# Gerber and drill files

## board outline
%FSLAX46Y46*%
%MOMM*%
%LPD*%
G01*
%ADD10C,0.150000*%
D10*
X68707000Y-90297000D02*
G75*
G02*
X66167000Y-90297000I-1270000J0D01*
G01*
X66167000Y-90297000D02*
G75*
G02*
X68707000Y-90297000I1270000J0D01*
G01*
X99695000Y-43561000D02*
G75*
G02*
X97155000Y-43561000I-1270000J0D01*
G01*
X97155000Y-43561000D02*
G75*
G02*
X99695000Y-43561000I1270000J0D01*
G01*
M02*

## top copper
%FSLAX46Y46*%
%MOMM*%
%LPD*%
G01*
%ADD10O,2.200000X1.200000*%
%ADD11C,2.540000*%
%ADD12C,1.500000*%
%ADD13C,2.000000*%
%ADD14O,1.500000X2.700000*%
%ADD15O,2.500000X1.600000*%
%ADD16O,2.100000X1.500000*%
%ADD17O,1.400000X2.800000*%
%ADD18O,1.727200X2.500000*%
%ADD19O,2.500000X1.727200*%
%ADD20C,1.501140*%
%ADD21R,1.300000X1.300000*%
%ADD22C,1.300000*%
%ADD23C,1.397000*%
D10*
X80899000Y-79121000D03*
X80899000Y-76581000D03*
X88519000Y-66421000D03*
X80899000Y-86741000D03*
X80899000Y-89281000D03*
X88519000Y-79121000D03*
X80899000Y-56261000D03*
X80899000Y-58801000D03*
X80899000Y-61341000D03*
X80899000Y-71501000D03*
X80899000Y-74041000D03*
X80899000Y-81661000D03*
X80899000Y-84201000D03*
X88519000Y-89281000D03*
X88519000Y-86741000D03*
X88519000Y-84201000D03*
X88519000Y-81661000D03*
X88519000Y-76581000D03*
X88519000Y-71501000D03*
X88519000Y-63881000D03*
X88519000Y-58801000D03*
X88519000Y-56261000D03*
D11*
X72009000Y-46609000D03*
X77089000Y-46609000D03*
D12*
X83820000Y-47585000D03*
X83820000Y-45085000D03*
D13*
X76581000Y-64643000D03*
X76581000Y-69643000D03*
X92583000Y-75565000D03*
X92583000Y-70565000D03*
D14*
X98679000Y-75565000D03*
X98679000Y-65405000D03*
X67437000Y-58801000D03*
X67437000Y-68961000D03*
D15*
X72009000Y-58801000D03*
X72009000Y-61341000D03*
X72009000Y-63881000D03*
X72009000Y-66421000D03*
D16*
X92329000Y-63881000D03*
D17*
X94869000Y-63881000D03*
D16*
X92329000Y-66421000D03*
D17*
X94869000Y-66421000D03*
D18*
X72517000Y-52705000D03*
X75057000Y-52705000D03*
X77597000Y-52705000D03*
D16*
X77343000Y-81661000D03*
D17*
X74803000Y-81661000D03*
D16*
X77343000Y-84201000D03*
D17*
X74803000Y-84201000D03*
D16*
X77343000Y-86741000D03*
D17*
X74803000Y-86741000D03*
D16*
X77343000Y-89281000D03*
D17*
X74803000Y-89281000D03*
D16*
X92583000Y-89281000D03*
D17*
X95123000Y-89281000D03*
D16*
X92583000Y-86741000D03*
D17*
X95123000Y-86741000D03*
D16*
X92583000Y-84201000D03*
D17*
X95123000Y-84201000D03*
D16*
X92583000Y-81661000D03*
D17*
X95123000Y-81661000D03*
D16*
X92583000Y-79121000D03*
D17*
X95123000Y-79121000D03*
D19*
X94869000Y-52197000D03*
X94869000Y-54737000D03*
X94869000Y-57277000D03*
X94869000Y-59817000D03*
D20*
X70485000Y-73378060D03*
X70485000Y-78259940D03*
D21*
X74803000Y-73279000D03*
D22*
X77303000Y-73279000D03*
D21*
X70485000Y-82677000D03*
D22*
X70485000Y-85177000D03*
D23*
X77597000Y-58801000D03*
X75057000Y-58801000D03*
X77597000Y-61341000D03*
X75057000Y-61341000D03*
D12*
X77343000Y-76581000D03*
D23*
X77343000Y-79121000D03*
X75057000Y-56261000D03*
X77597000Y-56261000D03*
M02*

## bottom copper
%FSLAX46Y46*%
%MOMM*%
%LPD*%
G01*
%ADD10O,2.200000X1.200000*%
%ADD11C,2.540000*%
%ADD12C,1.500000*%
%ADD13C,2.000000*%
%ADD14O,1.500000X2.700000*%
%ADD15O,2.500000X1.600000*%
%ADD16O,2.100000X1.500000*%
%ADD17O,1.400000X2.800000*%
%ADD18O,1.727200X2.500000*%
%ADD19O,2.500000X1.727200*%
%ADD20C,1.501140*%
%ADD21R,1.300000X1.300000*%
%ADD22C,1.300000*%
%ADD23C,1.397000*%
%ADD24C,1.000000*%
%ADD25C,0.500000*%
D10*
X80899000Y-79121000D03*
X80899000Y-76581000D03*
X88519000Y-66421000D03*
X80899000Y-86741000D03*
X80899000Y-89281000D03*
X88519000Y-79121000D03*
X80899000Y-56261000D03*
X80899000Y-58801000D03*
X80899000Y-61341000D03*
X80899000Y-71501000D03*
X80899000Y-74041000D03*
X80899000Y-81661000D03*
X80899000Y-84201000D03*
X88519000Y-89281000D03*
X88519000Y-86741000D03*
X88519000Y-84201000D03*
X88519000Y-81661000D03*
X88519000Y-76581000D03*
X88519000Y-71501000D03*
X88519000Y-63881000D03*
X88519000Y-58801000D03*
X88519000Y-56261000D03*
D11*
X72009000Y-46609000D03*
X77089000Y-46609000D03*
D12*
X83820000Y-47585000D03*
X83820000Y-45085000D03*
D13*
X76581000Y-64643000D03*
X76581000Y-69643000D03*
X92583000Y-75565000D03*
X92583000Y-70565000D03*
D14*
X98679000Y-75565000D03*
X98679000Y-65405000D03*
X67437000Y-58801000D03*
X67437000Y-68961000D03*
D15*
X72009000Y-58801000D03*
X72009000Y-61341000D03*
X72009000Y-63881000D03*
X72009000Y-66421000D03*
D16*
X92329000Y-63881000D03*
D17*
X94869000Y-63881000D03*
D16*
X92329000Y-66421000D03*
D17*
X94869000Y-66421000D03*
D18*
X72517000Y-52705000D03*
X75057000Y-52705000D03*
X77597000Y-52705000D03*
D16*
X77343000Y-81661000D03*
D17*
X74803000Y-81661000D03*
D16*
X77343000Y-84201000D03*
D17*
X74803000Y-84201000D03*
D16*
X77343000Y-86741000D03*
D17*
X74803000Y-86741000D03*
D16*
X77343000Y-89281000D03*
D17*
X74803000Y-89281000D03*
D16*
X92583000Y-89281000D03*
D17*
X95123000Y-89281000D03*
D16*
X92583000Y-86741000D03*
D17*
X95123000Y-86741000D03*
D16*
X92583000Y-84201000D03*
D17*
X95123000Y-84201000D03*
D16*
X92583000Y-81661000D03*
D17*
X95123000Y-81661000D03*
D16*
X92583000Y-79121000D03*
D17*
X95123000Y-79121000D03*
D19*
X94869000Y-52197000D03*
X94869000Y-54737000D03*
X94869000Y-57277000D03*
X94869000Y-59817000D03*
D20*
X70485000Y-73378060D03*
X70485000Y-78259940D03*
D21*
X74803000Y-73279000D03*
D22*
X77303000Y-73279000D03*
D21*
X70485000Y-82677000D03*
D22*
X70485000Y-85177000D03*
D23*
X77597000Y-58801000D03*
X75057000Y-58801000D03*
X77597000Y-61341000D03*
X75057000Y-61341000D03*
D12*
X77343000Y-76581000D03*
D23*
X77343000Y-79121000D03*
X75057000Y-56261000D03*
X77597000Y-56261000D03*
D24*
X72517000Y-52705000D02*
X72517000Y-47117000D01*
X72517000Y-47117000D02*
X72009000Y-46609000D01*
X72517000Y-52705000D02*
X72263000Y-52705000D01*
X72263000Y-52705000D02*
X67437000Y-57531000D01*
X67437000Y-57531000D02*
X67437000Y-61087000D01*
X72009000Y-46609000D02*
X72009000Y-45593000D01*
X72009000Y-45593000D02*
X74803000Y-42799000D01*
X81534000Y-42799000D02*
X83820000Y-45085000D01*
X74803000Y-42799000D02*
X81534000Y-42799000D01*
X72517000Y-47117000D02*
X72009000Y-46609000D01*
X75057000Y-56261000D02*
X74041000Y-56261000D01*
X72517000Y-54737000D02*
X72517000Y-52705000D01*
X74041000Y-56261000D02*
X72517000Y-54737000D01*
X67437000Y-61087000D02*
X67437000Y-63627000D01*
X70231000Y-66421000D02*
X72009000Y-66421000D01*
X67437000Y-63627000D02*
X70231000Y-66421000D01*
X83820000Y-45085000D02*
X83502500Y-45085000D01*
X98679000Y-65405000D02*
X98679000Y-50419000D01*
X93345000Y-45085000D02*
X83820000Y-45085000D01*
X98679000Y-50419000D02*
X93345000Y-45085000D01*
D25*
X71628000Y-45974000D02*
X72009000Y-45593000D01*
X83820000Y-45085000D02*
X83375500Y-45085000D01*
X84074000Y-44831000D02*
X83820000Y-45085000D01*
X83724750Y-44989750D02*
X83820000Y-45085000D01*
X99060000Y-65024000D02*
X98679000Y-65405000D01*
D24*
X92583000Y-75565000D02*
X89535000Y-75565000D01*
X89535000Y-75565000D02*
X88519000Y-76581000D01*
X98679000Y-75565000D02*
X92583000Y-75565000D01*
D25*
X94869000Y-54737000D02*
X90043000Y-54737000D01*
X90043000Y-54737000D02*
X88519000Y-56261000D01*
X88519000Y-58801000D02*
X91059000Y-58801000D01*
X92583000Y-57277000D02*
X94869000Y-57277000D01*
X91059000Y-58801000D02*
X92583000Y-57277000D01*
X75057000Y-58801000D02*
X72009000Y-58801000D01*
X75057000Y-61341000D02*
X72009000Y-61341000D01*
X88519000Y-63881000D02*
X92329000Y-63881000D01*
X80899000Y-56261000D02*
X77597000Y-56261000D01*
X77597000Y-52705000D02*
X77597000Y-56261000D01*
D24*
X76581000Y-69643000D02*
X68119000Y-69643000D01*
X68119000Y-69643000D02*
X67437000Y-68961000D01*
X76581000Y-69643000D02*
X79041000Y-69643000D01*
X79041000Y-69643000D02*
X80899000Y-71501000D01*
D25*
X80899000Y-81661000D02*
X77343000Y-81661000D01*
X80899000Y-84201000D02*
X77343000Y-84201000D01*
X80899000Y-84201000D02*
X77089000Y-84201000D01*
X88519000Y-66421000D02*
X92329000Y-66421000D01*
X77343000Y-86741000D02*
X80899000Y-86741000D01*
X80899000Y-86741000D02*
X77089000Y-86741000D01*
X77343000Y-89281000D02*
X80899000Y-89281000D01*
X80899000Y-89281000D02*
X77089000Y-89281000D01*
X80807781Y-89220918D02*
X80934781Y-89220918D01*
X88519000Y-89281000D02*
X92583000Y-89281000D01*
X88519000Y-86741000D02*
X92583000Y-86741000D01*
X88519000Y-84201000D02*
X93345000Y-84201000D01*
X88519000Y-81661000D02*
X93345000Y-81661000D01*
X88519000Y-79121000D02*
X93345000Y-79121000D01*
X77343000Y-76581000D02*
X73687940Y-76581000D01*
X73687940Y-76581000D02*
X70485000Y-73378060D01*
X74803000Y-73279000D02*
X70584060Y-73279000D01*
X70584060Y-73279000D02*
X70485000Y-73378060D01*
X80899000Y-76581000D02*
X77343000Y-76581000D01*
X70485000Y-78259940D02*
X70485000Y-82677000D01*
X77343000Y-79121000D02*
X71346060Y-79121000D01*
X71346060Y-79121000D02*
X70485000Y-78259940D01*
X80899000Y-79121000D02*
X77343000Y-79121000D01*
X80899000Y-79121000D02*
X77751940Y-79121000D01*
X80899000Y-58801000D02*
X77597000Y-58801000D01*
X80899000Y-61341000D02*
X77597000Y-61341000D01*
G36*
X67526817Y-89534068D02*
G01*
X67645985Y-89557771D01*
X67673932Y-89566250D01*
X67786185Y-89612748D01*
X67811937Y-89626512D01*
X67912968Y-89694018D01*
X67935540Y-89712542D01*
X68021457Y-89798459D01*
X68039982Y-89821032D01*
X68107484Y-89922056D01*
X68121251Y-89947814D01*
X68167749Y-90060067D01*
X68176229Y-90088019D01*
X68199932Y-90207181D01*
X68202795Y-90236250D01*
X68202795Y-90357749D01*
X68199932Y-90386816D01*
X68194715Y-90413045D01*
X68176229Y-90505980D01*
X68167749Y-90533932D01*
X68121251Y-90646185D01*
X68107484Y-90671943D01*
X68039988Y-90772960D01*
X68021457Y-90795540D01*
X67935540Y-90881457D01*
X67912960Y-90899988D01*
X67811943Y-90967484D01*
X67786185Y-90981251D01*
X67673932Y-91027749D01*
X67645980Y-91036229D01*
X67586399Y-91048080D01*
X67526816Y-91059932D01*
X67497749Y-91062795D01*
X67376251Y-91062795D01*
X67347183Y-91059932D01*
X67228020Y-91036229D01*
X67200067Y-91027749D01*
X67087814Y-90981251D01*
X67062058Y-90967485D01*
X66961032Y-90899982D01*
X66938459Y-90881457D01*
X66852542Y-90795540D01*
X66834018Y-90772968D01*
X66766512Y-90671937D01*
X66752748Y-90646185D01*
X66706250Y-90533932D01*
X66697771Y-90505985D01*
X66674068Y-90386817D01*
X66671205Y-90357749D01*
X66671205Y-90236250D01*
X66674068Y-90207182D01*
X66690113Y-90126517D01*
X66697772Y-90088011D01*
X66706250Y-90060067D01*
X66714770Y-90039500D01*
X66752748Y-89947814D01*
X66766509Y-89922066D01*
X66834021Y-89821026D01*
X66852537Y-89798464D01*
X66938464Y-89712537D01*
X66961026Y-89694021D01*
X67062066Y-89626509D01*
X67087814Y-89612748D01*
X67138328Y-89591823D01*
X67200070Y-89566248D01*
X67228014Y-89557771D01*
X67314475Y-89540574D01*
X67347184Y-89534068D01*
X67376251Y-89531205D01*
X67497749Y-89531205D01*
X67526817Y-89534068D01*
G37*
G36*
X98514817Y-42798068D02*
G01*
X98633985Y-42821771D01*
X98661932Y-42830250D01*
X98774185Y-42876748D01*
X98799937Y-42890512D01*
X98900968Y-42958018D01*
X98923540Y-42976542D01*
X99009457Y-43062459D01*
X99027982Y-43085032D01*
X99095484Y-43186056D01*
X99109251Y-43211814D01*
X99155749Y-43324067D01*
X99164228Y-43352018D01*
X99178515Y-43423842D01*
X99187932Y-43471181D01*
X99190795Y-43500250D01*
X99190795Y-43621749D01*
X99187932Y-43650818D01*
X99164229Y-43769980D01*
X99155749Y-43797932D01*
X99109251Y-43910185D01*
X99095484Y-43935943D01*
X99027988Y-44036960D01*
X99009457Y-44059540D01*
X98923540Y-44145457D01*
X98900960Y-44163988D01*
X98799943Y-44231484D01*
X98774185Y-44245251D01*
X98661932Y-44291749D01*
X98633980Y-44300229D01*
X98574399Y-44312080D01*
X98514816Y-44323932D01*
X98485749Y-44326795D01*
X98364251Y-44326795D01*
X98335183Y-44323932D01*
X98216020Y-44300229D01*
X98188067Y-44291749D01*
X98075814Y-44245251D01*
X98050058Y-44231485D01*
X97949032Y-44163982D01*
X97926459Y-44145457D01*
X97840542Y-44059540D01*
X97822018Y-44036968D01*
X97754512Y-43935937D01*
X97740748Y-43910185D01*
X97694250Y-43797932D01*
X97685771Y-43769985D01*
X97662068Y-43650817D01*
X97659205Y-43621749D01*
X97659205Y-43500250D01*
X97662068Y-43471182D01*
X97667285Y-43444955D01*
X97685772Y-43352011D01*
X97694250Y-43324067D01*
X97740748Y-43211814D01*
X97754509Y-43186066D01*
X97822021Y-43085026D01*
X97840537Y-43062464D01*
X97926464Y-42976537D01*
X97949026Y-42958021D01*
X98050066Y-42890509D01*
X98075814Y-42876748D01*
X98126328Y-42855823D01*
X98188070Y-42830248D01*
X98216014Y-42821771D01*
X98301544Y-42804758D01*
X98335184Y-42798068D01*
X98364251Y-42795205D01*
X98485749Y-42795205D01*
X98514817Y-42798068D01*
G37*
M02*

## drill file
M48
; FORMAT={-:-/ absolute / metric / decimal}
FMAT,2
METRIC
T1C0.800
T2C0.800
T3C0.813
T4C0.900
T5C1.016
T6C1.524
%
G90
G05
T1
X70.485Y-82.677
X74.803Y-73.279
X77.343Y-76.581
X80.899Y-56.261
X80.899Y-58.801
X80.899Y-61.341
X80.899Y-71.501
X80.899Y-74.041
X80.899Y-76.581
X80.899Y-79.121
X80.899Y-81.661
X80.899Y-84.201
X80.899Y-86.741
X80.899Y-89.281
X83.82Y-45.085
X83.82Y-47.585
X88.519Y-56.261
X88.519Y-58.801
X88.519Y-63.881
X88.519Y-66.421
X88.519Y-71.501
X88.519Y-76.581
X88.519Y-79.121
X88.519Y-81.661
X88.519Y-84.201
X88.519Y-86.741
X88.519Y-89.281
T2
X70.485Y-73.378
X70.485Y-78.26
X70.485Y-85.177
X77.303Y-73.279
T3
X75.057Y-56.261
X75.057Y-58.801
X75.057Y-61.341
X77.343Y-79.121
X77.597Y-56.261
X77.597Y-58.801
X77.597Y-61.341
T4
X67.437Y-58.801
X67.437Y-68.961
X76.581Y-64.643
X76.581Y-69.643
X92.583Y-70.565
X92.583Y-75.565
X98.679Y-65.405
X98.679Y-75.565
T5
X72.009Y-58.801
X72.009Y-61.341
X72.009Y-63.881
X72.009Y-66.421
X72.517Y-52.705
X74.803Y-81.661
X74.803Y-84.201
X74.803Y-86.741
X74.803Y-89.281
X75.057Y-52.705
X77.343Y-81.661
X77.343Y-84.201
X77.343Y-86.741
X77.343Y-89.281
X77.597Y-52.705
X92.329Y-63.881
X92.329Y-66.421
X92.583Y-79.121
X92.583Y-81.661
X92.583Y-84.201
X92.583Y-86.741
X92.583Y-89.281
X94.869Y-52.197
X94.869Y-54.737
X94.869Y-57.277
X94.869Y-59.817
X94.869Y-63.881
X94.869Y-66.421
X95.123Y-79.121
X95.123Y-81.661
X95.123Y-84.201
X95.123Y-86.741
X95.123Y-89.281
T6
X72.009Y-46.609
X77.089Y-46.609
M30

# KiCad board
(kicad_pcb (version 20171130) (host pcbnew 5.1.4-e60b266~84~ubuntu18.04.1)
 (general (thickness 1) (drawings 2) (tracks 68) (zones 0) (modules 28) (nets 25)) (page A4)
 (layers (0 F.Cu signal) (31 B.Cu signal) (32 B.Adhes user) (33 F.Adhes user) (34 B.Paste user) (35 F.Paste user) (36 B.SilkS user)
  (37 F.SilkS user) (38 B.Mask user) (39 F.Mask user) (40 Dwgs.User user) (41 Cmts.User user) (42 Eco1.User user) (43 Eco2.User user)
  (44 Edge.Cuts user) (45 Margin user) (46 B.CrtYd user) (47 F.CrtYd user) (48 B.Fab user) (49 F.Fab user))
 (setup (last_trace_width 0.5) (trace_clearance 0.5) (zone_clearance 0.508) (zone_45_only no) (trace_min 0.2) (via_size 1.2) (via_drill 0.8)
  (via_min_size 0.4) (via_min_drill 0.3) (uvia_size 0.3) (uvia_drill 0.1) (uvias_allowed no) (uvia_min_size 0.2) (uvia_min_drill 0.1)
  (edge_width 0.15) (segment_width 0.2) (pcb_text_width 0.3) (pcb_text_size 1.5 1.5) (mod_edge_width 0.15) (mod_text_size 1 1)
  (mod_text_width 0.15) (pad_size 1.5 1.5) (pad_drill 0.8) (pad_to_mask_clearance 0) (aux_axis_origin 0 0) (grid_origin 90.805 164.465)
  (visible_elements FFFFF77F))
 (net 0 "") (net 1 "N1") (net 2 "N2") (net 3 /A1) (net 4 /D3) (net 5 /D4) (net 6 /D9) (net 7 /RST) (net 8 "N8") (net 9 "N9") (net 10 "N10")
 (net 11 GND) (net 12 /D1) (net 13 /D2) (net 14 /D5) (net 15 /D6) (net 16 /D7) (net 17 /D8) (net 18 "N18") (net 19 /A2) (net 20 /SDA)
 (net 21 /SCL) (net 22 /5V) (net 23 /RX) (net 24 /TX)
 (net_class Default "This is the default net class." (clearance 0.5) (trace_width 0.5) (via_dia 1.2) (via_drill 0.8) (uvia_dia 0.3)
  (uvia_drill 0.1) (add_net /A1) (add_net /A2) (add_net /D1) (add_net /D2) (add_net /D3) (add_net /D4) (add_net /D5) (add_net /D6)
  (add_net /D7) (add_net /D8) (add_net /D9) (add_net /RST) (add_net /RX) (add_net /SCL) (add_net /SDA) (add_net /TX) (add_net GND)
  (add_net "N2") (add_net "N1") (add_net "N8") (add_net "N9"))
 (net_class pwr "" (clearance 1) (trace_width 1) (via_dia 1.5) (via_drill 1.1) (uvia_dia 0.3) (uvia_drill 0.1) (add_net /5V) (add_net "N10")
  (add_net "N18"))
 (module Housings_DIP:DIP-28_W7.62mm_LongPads (layer F.Cu) (at 80.899 56.261)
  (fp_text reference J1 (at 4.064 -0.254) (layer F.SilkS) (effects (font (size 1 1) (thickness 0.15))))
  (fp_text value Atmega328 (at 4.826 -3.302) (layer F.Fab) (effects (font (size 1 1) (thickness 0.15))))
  (pad 10 thru_hole oval (at 0 22.86) (size 2.2 1.2) (drill 0.8) (layers *.Cu *.Mask F.SilkS) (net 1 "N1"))
  (pad 9 thru_hole oval (at 0 20.32) (size 2.2 1.2) (drill 0.8) (layers *.Cu *.Mask F.SilkS) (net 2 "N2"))
  (pad 24 thru_hole oval (at 7.62 10.16) (size 2.2 1.2) (drill 0.8) (layers *.Cu *.Mask F.SilkS) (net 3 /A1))
  (pad 13 thru_hole oval (at 0 30.48) (size 2.2 1.2) (drill 0.8) (layers *.Cu *.Mask F.SilkS) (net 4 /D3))
  (pad 14 thru_hole oval (at 0 33.02) (size 2.2 1.2) (drill 0.8) (layers *.Cu *.Mask F.SilkS) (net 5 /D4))
  (pad 19 thru_hole oval (at 7.62 22.86) (size 2.2 1.2) (drill 0.8) (layers *.Cu *.Mask F.SilkS) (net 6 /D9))
  (pad 1 thru_hole oval (at 0 0) (size 2.2 1.2) (drill 0.8) (layers *.Cu *.Mask F.SilkS) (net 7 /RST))
  (pad 2 thru_hole oval (at 0 2.54) (size 2.2 1.2) (drill 0.8) (layers *.Cu *.Mask F.SilkS) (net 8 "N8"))
  (pad 3 thru_hole oval (at 0 5.08) (size 2.2 1.2) (drill 0.8) (layers *.Cu *.Mask F.SilkS) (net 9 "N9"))
  (pad 7 thru_hole oval (at 0 15.24) (size 2.2 1.2) (drill 0.8) (layers *.Cu *.Mask F.SilkS) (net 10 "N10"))
  (pad 8 thru_hole oval (at 0 17.78) (size 2.2 1.2) (drill 0.8) (layers *.Cu *.Mask F.SilkS) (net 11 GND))
  (pad 11 thru_hole oval (at 0 25.4) (size 2.2 1.2) (drill 0.8) (layers *.Cu *.Mask F.SilkS) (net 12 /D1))
  (pad 12 thru_hole oval (at 0 27.94) (size 2.2 1.2) (drill 0.8) (layers *.Cu *.Mask F.SilkS) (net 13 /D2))
  (pad 15 thru_hole oval (at 7.62 33.02) (size 2.2 1.2) (drill 0.8) (layers *.Cu *.Mask F.SilkS) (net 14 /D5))
  (pad 16 thru_hole oval (at 7.62 30.48) (size 2.2 1.2) (drill 0.8) (layers *.Cu *.Mask F.SilkS) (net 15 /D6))
  (pad 17 thru_hole oval (at 7.62 27.94) (size 2.2 1.2) (drill 0.8) (layers *.Cu *.Mask F.SilkS) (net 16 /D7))
  (pad 18 thru_hole oval (at 7.62 25.4) (size 2.2 1.2) (drill 0.8) (layers *.Cu *.Mask F.SilkS) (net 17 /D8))
  (pad 20 thru_hole oval (at 7.62 20.32) (size 2.2 1.2) (drill 0.8) (layers *.Cu *.Mask F.SilkS) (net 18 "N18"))
  (pad 22 thru_hole oval (at 7.62 15.24) (size 2.2 1.2) (drill 0.8) (layers *.Cu *.Mask F.SilkS) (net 11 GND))
  (pad 25 thru_hole oval (at 7.62 7.62) (size 2.2 1.2) (drill 0.8) (layers *.Cu *.Mask F.SilkS) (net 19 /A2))
  (pad 27 thru_hole oval (at 7.62 2.54) (size 2.2 1.2) (drill 0.8) (layers *.Cu *.Mask F.SilkS) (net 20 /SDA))
  (pad 28 thru_hole oval (at 7.62 0) (size 2.2 1.2) (drill 0.8) (layers *.Cu *.Mask F.SilkS) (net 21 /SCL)))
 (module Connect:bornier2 (layer F.Cu) (at 74.549 46.609)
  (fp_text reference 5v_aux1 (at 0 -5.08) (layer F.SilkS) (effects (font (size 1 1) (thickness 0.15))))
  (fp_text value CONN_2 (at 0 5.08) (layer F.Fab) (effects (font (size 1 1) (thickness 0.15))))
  (pad 1 thru_hole circle (at -2.54 0) (size 2.54 2.54) (drill 1.524) (layers *.Cu *.Mask F.SilkS) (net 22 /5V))
  (pad 2 thru_hole circle (at 2.54 0) (size 2.54 2.54) (drill 1.524) (layers *.Cu *.Mask F.SilkS) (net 11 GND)))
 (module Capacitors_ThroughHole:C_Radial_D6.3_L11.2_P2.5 (layer F.Cu) (at 83.82 45.085 270)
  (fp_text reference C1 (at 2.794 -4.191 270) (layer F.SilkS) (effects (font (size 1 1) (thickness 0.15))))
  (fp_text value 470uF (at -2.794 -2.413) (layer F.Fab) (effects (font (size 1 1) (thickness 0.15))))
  (pad 2 thru_hole circle (at 2.5 0 270) (size 1.5 1.5) (drill 0.8) (layers *.Cu *.Mask F.SilkS) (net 11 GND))
  (pad 1 thru_hole circle (at 0 0 270) (size 1.5 1.5) (drill 0.8) (layers *.Cu *.Mask F.SilkS) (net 22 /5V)))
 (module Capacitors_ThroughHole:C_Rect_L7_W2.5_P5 (layer F.Cu) (at 76.581 64.643 270)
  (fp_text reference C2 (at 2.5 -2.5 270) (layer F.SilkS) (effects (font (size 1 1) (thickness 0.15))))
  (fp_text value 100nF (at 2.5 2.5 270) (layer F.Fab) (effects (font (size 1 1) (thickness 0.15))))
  (pad 1 thru_hole circle (at 0 0 270) (size 2 2) (drill 0.9) (layers *.Cu *.Mask F.SilkS) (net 11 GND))
  (pad 2 thru_hole circle (at 5 0 270) (size 2 2) (drill 0.9) (layers *.Cu *.Mask F.SilkS) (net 10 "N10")))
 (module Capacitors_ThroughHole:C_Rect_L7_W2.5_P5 (layer F.Cu) (at 92.583 75.565 90)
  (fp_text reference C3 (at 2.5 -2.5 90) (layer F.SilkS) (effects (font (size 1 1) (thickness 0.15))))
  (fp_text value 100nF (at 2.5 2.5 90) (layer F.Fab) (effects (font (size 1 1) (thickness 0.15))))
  (pad 1 thru_hole circle (at 0 0 90) (size 2 2) (drill 0.9) (layers *.Cu *.Mask F.SilkS) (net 18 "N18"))
  (pad 2 thru_hole circle (at 5 0 90) (size 2 2) (drill 0.9) (layers *.Cu *.Mask F.SilkS) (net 11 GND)))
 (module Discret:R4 (layer F.Cu) (at 98.679 70.485 90)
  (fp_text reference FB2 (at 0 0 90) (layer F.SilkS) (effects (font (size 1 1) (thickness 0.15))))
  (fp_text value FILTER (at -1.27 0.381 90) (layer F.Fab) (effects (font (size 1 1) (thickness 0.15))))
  (pad 1 thru_hole oval (at -5.08 0 90) (size 2.7 1.5) (drill 0.9) (layers *.Cu *.Mask F.SilkS) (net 18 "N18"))
  (pad 2 thru_hole oval (at 5.08 0 90) (size 2.7 1.5) (drill 0.9) (layers *.Cu *.Mask F.SilkS) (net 22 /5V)))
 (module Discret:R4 (layer F.Cu) (at 67.437 63.881 270)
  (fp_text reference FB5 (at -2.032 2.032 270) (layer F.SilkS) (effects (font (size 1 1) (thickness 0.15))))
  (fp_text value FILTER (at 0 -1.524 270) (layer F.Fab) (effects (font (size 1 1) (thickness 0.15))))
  (pad 1 thru_hole oval (at -5.08 0 270) (size 2.7 1.5) (drill 0.9) (layers *.Cu *.Mask F.SilkS) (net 22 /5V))
  (pad 2 thru_hole oval (at 5.08 0 270) (size 2.7 1.5) (drill 0.9) (layers *.Cu *.Mask F.SilkS) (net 10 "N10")))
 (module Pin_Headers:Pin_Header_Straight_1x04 (layer F.Cu) (at 72.009 58.801)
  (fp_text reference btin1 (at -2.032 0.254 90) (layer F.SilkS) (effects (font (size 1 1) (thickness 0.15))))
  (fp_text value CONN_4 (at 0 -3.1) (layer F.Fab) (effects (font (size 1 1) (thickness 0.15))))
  (pad 1 thru_hole oval (at 0 0) (size 2.5 1.6) (drill 1.016) (layers *.Cu *.Mask F.SilkS) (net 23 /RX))
  (pad 2 thru_hole oval (at 0 2.54) (size 2.5 1.6) (drill 1.016) (layers *.Cu *.Mask F.SilkS) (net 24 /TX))
  (pad 3 thru_hole oval (at 0 5.08) (size 2.5 1.6) (drill 1.016) (layers *.Cu *.Mask F.SilkS) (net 11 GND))
  (pad 4 thru_hole oval (at 0 7.62) (size 2.5 1.6) (drill 1.016) (layers *.Cu *.Mask F.SilkS) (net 22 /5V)))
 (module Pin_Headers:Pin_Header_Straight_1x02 (layer F.Cu) (at 92.329 63.881 90)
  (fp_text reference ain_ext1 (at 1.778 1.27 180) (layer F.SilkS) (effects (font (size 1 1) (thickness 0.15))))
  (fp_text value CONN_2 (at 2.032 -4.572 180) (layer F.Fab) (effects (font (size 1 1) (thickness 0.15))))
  (pad 1 thru_hole oval (at 0 0 90) (size 1.5 2.1) (drill 1.016) (layers *.Cu *.Mask F.SilkS) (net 19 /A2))
  (pad 2 thru_hole oval (at 0 2.54 90) (size 2.8 1.4) (drill 1.016) (layers *.Cu *.Mask F.SilkS) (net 11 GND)))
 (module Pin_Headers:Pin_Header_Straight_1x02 (layer F.Cu) (at 92.329 66.421 90)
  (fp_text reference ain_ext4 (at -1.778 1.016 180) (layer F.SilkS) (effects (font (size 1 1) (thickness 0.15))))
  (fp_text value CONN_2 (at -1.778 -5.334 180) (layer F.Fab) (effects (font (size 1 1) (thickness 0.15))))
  (pad 1 thru_hole oval (at 0 0 90) (size 1.5 2.1) (drill 1.016) (layers *.Cu *.Mask F.SilkS) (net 3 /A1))
  (pad 2 thru_hole oval (at 0 2.54 90) (size 2.8 1.4) (drill 1.016) (layers *.Cu *.Mask F.SilkS) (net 11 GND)))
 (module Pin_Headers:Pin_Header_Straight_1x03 (layer F.Cu) (at 72.517 52.705 90)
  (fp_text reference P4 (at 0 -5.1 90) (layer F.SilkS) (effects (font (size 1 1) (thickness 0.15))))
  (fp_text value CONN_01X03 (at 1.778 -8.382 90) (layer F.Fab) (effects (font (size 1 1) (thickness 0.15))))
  (pad 1 thru_hole oval (at 0 0 90) (size 2.5 1.7272) (drill 1.016) (layers *.Cu *.Mask F.SilkS) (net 22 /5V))
  (pad 2 thru_hole oval (at 0 2.54 90) (size 2.5 1.7272) (drill 1.016) (layers *.Cu *.Mask F.SilkS) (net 11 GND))
  (pad 3 thru_hole oval (at 0 5.08 90) (size 2.5 1.7272) (drill 1.016) (layers *.Cu *.Mask F.SilkS) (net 7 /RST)))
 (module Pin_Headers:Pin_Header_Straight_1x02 (layer F.Cu) (at 77.343 81.661 270)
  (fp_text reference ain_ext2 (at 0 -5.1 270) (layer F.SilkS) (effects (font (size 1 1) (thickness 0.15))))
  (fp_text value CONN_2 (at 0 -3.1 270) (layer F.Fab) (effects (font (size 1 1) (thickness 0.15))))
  (pad 1 thru_hole oval (at 0 0 270) (size 1.5 2.1) (drill 1.016) (layers *.Cu *.Mask F.SilkS) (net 12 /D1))
  (pad 2 thru_hole oval (at 0 2.54 270) (size 2.8 1.4) (drill 1.016) (layers *.Cu *.Mask F.SilkS) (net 11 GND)))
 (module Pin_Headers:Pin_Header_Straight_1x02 (layer F.Cu) (at 77.343 84.201 270)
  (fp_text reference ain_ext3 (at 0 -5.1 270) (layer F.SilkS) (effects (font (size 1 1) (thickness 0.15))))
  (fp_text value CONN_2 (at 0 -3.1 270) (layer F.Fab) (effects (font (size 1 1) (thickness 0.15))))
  (pad 1 thru_hole oval (at 0 0 270) (size 1.5 2.1) (drill 1.016) (layers *.Cu *.Mask F.SilkS) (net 13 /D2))
  (pad 2 thru_hole oval (at 0 2.54 270) (size 2.8 1.4) (drill 1.016) (layers *.Cu *.Mask F.SilkS) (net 11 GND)))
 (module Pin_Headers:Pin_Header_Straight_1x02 (layer F.Cu) (at 77.343 86.741 270)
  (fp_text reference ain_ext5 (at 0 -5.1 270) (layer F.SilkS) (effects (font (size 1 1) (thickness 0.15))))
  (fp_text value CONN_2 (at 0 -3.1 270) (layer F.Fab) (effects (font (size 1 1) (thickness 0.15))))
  (pad 1 thru_hole oval (at 0 0 270) (size 1.5 2.1) (drill 1.016) (layers *.Cu *.Mask F.SilkS) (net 4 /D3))
  (pad 2 thru_hole oval (at 0 2.54 270) (size 2.8 1.4) (drill 1.016) (layers *.Cu *.Mask F.SilkS) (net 11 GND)))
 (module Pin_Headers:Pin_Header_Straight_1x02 (layer F.Cu) (at 77.343 89.281 270)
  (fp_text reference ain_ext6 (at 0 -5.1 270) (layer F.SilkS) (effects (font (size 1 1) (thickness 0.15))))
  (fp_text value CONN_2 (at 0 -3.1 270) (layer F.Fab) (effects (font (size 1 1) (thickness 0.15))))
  (pad 1 thru_hole oval (at 0 0 270) (size 1.5 2.1) (drill 1.016) (layers *.Cu *.Mask F.SilkS) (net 5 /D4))
  (pad 2 thru_hole oval (at 0 2.54 270) (size 2.8 1.4) (drill 1.016) (layers *.Cu *.Mask F.SilkS) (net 11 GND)))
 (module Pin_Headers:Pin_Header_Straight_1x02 (layer F.Cu) (at 92.583 89.281 90)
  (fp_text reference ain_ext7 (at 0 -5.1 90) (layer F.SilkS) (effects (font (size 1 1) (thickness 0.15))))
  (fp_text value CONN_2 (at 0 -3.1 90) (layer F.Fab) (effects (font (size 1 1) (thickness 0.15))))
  (pad 1 thru_hole oval (at 0 0 90) (size 1.5 2.1) (drill 1.016) (layers *.Cu *.Mask F.SilkS) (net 14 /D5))
  (pad 2 thru_hole oval (at 0 2.54 90) (size 2.8 1.4) (drill 1.016) (layers *.Cu *.Mask F.SilkS) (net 11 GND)))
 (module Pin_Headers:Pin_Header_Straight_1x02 (layer F.Cu) (at 92.583 86.741 90)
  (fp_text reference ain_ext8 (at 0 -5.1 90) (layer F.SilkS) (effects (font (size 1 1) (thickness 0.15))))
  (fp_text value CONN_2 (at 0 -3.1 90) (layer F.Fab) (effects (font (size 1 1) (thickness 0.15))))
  (pad 1 thru_hole oval (at 0 0 90) (size 1.5 2.1) (drill 1.016) (layers *.Cu *.Mask F.SilkS) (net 15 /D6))
  (pad 2 thru_hole oval (at 0 2.54 90) (size 2.8 1.4) (drill 1.016) (layers *.Cu *.Mask F.SilkS) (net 11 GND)))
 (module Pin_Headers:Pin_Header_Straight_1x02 (layer F.Cu) (at 92.583 84.201 90)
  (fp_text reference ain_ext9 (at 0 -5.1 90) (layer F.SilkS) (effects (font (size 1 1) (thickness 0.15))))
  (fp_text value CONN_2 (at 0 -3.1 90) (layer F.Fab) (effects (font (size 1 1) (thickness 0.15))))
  (pad 1 thru_hole oval (at 0 0 90) (size 1.5 2.1) (drill 1.016) (layers *.Cu *.Mask F.SilkS) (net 16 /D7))
  (pad 2 thru_hole oval (at 0 2.54 90) (size 2.8 1.4) (drill 1.016) (layers *.Cu *.Mask F.SilkS) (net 11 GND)))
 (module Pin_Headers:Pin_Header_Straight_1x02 (layer F.Cu) (at 92.583 81.661 90)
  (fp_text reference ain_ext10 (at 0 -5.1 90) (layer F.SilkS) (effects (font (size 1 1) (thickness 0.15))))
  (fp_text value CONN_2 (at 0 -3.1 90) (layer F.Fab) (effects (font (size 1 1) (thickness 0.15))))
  (pad 1 thru_hole oval (at 0 0 90) (size 1.5 2.1) (drill 1.016) (layers *.Cu *.Mask F.SilkS) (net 17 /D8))
  (pad 2 thru_hole oval (at 0 2.54 90) (size 2.8 1.4) (drill 1.016) (layers *.Cu *.Mask F.SilkS) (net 11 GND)))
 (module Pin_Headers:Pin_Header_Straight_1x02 (layer F.Cu) (at 92.583 79.121 90)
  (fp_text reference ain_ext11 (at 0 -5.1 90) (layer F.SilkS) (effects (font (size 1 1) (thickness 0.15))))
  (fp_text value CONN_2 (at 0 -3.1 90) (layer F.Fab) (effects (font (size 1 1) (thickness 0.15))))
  (pad 1 thru_hole oval (at 0 0 90) (size 1.5 2.1) (drill 1.016) (layers *.Cu *.Mask F.SilkS) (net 6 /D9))
  (pad 2 thru_hole oval (at 0 2.54 90) (size 2.8 1.4) (drill 1.016) (layers *.Cu *.Mask F.SilkS) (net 11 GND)))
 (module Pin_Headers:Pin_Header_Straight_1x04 (layer F.Cu) (at 94.869 52.197)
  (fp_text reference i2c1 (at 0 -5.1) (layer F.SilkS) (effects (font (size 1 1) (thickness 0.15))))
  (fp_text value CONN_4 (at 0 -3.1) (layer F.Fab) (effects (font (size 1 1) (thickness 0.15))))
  (pad 1 thru_hole oval (at 0 0) (size 2.5 1.7272) (drill 1.016) (layers *.Cu *.Mask F.SilkS) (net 11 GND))
  (pad 2 thru_hole oval (at 0 2.54) (size 2.5 1.7272) (drill 1.016) (layers *.Cu *.Mask F.SilkS) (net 21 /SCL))
  (pad 3 thru_hole oval (at 0 5.08) (size 2.5 1.7272) (drill 1.016) (layers *.Cu *.Mask F.SilkS) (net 20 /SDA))
  (pad 4 thru_hole oval (at 0 7.62) (size 2.5 1.7272) (drill 1.016) (layers *.Cu *.Mask F.SilkS) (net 11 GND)))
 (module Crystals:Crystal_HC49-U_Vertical (layer F.Cu) (at 70.485 75.819 270)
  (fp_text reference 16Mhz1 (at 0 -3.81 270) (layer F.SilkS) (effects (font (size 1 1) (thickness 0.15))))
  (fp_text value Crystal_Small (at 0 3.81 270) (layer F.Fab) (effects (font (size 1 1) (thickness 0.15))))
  (pad 1 thru_hole circle (at -2.44094 0 270) (size 1.50114 1.50114) (drill 0.8001) (layers *.Cu *.Mask F.SilkS) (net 2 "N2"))
  (pad 2 thru_hole circle (at 2.44094 0 270) (size 1.50114 1.50114) (drill 0.8001) (layers *.Cu *.Mask F.SilkS) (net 1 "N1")))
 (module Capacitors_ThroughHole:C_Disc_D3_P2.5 (layer F.Cu) (at 74.803 73.279)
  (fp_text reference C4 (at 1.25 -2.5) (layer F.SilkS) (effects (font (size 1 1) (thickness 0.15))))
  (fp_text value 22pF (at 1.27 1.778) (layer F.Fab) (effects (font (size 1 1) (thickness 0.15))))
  (pad 1 thru_hole rect (at 0 0) (size 1.3 1.3) (drill 0.8) (layers *.Cu *.Mask F.SilkS) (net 2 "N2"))
  (pad 2 thru_hole circle (at 2.5 0) (size 1.3 1.3) (drill 0.8001) (layers *.Cu *.Mask F.SilkS) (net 11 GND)))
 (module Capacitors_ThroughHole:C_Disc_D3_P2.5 (layer F.Cu) (at 70.485 82.677 270)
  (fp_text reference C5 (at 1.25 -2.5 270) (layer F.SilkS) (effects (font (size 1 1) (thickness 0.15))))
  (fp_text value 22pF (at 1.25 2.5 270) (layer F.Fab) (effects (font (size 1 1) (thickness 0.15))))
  (pad 1 thru_hole rect (at 0 0 270) (size 1.3 1.3) (drill 0.8) (layers *.Cu *.Mask F.SilkS) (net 1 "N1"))
  (pad 2 thru_hole circle (at 2.5 0 270) (size 1.3 1.3) (drill 0.8001) (layers *.Cu *.Mask F.SilkS) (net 11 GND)))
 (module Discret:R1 (layer F.Cu) (at 76.327 58.801 180)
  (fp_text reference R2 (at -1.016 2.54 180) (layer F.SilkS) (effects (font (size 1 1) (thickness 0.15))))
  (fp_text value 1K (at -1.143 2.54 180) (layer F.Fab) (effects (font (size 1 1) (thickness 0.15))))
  (pad 1 thru_hole circle (at -1.27 0 180) (size 1.397 1.397) (drill 0.8128) (layers *.Cu *.Mask F.SilkS) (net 8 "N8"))
  (pad 2 thru_hole circle (at 1.27 0 180) (size 1.397 1.397) (drill 0.8128) (layers *.Cu *.Mask F.SilkS) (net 23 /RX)))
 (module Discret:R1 (layer F.Cu) (at 76.327 61.341 180)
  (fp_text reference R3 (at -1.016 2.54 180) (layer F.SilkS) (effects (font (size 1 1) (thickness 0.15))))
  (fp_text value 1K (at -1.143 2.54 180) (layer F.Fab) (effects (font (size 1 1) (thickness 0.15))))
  (pad 1 thru_hole circle (at -1.27 0 180) (size 1.397 1.397) (drill 0.8128) (layers *.Cu *.Mask F.SilkS) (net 9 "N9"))
  (pad 2 thru_hole circle (at 1.27 0 180) (size 1.397 1.397) (drill 0.8128) (layers *.Cu *.Mask F.SilkS) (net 24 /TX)))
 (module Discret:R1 (layer F.Cu) (at 77.343 77.851 270)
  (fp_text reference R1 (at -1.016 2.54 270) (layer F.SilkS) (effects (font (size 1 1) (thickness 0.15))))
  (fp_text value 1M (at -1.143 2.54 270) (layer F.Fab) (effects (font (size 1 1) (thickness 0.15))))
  (pad 1 thru_hole circle (at -1.27 0 270) (size 1.5 1.5) (drill 0.8) (layers *.Cu *.Mask F.SilkS) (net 2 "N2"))
  (pad 2 thru_hole circle (at 1.27 0 270) (size 1.397 1.397) (drill 0.8128) (layers *.Cu *.Mask F.SilkS) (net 1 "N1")))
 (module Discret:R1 (layer F.Cu) (at 76.327 56.261)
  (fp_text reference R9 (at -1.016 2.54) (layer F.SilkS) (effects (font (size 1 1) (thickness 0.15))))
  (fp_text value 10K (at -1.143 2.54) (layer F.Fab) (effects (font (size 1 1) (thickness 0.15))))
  (pad 1 thru_hole circle (at -1.27 0) (size 1.397 1.397) (drill 0.8128) (layers *.Cu *.Mask F.SilkS) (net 22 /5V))
  (pad 2 thru_hole circle (at 1.27 0) (size 1.397 1.397) (drill 0.8128) (layers *.Cu *.Mask F.SilkS) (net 7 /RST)))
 (gr_circle (center 67.437 90.297) (end 68.707 90.297) (layer Edge.Cuts) (width 0.15))
 (gr_circle (center 98.425 43.561) (end 99.695 43.561) (layer Edge.Cuts) (width 0.15))
 (segment (start 72.517 52.705) (end 72.517 47.117) (width 1) (layer B.Cu) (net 22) (status C00000))
 (segment (start 72.517 47.117) (end 72.009 46.609) (width 1) (layer B.Cu) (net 22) (status C00000))
 (segment (start 72.517 52.705) (end 72.263 52.705) (width 1) (layer B.Cu) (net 22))
 (segment (start 72.263 52.705) (end 67.437 57.531) (width 1) (layer B.Cu) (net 22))
 (segment (start 67.437 57.531) (end 67.437 61.087) (width 1) (layer B.Cu) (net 22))
 (segment (start 72.009 46.609) (end 72.009 45.593) (width 1) (layer B.Cu) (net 22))
 (segment (start 72.009 45.593) (end 74.803 42.799) (width 1) (layer B.Cu) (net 22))
 (segment (start 81.534 42.799) (end 83.82 45.085) (width 1) (layer B.Cu) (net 22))
 (segment (start 74.803 42.799) (end 81.534 42.799) (width 1) (layer B.Cu) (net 22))
 (segment (start 72.517 47.117) (end 72.009 46.609) (width 1) (layer B.Cu) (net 22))
 (segment (start 75.057 56.261) (end 74.041 56.261) (width 1) (layer B.Cu) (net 22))
 (segment (start 72.517 54.737) (end 72.517 52.705) (width 1) (layer B.Cu) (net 22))
 (segment (start 74.041 56.261) (end 72.517 54.737) (width 1) (layer B.Cu) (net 22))
 (segment (start 67.437 61.087) (end 67.437 63.627) (width 1) (layer B.Cu) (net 22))
 (segment (start 70.231 66.421) (end 72.009 66.421) (width 1) (layer B.Cu) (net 22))
 (segment (start 67.437 63.627) (end 70.231 66.421) (width 1) (layer B.Cu) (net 22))
 (segment (start 83.82 45.085) (end 83.5025 45.085) (width 1) (layer B.Cu) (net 22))
 (segment (start 98.679 65.405) (end 98.679 50.419) (width 1) (layer B.Cu) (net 22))
 (segment (start 93.345 45.085) (end 83.82 45.085) (width 1) (layer B.Cu) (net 22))
 (segment (start 98.679 50.419) (end 93.345 45.085) (width 1) (layer B.Cu) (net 22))
 (segment (start 71.628 45.974) (end 72.009 45.593) (width 0.5) (layer B.Cu) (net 22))
 (segment (start 83.82 45.085) (end 83.3755 45.085) (width 0.5) (layer B.Cu) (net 22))
 (segment (start 84.074 44.831) (end 83.82 45.085) (width 0.5) (layer B.Cu) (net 22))
 (segment (start 83.72475 44.98975) (end 83.82 45.085) (width 0.5) (layer B.Cu) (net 22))
 (segment (start 99.06 65.024) (end 98.679 65.405) (width 0.5) (layer B.Cu) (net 22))
 (segment (start 92.583 75.565) (end 89.535 75.565) (width 1) (layer B.Cu) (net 18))
 (segment (start 89.535 75.565) (end 88.519 76.581) (width 1) (layer B.Cu) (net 18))
 (segment (start 98.679 75.565) (end 92.583 75.565) (width 1) (layer B.Cu) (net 18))
 (segment (start 94.869 54.737) (end 90.043 54.737) (width 0.5) (layer B.Cu) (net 21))
 (segment (start 90.043 54.737) (end 88.519 56.261) (width 0.5) (layer B.Cu) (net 21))
 (segment (start 88.519 58.801) (end 91.059 58.801) (width 0.5) (layer B.Cu) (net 20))
 (segment (start 92.583 57.277) (end 94.869 57.277) (width 0.5) (layer B.Cu) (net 20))
 (segment (start 91.059 58.801) (end 92.583 57.277) (width 0.5) (layer B.Cu) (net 20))
 (segment (start 75.057 58.801) (end 72.009 58.801) (width 0.5) (layer B.Cu) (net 23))
 (segment (start 75.057 61.341) (end 72.009 61.341) (width 0.5) (layer B.Cu) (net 24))
 (segment (start 88.519 63.881) (end 92.329 63.881) (width 0.5) (layer B.Cu) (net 19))
 (segment (start 80.899 56.261) (end 77.597 56.261) (width 0.5) (layer B.Cu) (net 7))
 (segment (start 77.597 52.705) (end 77.597 56.261) (width 0.5) (layer B.Cu) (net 7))
 (segment (start 76.581 69.643) (end 68.119 69.643) (width 1) (layer B.Cu) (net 10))
 (segment (start 68.119 69.643) (end 67.437 68.961) (width 1) (layer B.Cu) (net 10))
 (segment (start 76.581 69.643) (end 79.041 69.643) (width 1) (layer B.Cu) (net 10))
 (segment (start 79.041 69.643) (end 80.899 71.501) (width 1) (layer B.Cu) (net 10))
 (segment (start 80.899 81.661) (end 77.343 81.661) (width 0.5) (layer B.Cu) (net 12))
 (segment (start 80.899 84.201) (end 77.343 84.201) (width 0.5) (layer B.Cu) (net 13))
 (segment (start 80.899 84.201) (end 77.089 84.201) (width 0.5) (layer B.Cu) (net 13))
 (segment (start 88.519 66.421) (end 92.329 66.421) (width 0.5) (layer B.Cu) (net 3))
 (segment (start 77.343 86.741) (end 80.899 86.741) (width 0.5) (layer B.Cu) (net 4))
 (segment (start 80.899 86.741) (end 77.089 86.741) (width 0.5) (layer B.Cu) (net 4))
 (segment (start 77.343 89.281) (end 80.899 89.281) (width 0.5) (layer B.Cu) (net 5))
 (segment (start 80.899 89.281) (end 77.089 89.281) (width 0.5) (layer B.Cu) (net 5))
 (segment (start 80.807781 89.220918) (end 80.934781 89.220918) (width 0.5) (layer B.Cu) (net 5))
 (segment (start 88.519 89.281) (end 92.583 89.281) (width 0.5) (layer B.Cu) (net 14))
 (segment (start 88.519 86.741) (end 92.583 86.741) (width 0.5) (layer B.Cu) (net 15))
 (segment (start 88.519 84.201) (end 93.345 84.201) (width 0.5) (layer B.Cu) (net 16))
 (segment (start 88.519 81.661) (end 93.345 81.661) (width 0.5) (layer B.Cu) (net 17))
 (segment (start 88.519 79.121) (end 93.345 79.121) (width 0.5) (layer B.Cu) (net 6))
 (segment (start 77.343 76.581) (end 73.68794 76.581) (width 0.5) (layer B.Cu) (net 2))
 (segment (start 73.68794 76.581) (end 70.485 73.37806) (width 0.5) (layer B.Cu) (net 2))
 (segment (start 74.803 73.279) (end 70.58406 73.279) (width 0.5) (layer B.Cu) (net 2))
 (segment (start 70.58406 73.279) (end 70.485 73.37806) (width 0.5) (layer B.Cu) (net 2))
 (segment (start 80.899 76.581) (end 77.343 76.581) (width 0.5) (layer B.Cu) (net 2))
 (segment (start 70.485 78.25994) (end 70.485 82.677) (width 0.5) (layer B.Cu) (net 1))
 (segment (start 77.343 79.121) (end 71.34606 79.121) (width 0.5) (layer B.Cu) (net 1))
 (segment (start 71.34606 79.121) (end 70.485 78.25994) (width 0.5) (layer B.Cu) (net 1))
 (segment (start 80.899 79.121) (end 77.343 79.121) (width 0.5) (layer B.Cu) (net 1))
 (segment (start 80.899 79.121) (end 77.75194 79.121) (width 0.5) (layer B.Cu) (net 1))
 (segment (start 80.899 58.801) (end 77.597 58.801) (width 0.5) (layer B.Cu) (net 8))
 (segment (start 80.899 61.341) (end 77.597 61.341) (width 0.5) (layer B.Cu) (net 9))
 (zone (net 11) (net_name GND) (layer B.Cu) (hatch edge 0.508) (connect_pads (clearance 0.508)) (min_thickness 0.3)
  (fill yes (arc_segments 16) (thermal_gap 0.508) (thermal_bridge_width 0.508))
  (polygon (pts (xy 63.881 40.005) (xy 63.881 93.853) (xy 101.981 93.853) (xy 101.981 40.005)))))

